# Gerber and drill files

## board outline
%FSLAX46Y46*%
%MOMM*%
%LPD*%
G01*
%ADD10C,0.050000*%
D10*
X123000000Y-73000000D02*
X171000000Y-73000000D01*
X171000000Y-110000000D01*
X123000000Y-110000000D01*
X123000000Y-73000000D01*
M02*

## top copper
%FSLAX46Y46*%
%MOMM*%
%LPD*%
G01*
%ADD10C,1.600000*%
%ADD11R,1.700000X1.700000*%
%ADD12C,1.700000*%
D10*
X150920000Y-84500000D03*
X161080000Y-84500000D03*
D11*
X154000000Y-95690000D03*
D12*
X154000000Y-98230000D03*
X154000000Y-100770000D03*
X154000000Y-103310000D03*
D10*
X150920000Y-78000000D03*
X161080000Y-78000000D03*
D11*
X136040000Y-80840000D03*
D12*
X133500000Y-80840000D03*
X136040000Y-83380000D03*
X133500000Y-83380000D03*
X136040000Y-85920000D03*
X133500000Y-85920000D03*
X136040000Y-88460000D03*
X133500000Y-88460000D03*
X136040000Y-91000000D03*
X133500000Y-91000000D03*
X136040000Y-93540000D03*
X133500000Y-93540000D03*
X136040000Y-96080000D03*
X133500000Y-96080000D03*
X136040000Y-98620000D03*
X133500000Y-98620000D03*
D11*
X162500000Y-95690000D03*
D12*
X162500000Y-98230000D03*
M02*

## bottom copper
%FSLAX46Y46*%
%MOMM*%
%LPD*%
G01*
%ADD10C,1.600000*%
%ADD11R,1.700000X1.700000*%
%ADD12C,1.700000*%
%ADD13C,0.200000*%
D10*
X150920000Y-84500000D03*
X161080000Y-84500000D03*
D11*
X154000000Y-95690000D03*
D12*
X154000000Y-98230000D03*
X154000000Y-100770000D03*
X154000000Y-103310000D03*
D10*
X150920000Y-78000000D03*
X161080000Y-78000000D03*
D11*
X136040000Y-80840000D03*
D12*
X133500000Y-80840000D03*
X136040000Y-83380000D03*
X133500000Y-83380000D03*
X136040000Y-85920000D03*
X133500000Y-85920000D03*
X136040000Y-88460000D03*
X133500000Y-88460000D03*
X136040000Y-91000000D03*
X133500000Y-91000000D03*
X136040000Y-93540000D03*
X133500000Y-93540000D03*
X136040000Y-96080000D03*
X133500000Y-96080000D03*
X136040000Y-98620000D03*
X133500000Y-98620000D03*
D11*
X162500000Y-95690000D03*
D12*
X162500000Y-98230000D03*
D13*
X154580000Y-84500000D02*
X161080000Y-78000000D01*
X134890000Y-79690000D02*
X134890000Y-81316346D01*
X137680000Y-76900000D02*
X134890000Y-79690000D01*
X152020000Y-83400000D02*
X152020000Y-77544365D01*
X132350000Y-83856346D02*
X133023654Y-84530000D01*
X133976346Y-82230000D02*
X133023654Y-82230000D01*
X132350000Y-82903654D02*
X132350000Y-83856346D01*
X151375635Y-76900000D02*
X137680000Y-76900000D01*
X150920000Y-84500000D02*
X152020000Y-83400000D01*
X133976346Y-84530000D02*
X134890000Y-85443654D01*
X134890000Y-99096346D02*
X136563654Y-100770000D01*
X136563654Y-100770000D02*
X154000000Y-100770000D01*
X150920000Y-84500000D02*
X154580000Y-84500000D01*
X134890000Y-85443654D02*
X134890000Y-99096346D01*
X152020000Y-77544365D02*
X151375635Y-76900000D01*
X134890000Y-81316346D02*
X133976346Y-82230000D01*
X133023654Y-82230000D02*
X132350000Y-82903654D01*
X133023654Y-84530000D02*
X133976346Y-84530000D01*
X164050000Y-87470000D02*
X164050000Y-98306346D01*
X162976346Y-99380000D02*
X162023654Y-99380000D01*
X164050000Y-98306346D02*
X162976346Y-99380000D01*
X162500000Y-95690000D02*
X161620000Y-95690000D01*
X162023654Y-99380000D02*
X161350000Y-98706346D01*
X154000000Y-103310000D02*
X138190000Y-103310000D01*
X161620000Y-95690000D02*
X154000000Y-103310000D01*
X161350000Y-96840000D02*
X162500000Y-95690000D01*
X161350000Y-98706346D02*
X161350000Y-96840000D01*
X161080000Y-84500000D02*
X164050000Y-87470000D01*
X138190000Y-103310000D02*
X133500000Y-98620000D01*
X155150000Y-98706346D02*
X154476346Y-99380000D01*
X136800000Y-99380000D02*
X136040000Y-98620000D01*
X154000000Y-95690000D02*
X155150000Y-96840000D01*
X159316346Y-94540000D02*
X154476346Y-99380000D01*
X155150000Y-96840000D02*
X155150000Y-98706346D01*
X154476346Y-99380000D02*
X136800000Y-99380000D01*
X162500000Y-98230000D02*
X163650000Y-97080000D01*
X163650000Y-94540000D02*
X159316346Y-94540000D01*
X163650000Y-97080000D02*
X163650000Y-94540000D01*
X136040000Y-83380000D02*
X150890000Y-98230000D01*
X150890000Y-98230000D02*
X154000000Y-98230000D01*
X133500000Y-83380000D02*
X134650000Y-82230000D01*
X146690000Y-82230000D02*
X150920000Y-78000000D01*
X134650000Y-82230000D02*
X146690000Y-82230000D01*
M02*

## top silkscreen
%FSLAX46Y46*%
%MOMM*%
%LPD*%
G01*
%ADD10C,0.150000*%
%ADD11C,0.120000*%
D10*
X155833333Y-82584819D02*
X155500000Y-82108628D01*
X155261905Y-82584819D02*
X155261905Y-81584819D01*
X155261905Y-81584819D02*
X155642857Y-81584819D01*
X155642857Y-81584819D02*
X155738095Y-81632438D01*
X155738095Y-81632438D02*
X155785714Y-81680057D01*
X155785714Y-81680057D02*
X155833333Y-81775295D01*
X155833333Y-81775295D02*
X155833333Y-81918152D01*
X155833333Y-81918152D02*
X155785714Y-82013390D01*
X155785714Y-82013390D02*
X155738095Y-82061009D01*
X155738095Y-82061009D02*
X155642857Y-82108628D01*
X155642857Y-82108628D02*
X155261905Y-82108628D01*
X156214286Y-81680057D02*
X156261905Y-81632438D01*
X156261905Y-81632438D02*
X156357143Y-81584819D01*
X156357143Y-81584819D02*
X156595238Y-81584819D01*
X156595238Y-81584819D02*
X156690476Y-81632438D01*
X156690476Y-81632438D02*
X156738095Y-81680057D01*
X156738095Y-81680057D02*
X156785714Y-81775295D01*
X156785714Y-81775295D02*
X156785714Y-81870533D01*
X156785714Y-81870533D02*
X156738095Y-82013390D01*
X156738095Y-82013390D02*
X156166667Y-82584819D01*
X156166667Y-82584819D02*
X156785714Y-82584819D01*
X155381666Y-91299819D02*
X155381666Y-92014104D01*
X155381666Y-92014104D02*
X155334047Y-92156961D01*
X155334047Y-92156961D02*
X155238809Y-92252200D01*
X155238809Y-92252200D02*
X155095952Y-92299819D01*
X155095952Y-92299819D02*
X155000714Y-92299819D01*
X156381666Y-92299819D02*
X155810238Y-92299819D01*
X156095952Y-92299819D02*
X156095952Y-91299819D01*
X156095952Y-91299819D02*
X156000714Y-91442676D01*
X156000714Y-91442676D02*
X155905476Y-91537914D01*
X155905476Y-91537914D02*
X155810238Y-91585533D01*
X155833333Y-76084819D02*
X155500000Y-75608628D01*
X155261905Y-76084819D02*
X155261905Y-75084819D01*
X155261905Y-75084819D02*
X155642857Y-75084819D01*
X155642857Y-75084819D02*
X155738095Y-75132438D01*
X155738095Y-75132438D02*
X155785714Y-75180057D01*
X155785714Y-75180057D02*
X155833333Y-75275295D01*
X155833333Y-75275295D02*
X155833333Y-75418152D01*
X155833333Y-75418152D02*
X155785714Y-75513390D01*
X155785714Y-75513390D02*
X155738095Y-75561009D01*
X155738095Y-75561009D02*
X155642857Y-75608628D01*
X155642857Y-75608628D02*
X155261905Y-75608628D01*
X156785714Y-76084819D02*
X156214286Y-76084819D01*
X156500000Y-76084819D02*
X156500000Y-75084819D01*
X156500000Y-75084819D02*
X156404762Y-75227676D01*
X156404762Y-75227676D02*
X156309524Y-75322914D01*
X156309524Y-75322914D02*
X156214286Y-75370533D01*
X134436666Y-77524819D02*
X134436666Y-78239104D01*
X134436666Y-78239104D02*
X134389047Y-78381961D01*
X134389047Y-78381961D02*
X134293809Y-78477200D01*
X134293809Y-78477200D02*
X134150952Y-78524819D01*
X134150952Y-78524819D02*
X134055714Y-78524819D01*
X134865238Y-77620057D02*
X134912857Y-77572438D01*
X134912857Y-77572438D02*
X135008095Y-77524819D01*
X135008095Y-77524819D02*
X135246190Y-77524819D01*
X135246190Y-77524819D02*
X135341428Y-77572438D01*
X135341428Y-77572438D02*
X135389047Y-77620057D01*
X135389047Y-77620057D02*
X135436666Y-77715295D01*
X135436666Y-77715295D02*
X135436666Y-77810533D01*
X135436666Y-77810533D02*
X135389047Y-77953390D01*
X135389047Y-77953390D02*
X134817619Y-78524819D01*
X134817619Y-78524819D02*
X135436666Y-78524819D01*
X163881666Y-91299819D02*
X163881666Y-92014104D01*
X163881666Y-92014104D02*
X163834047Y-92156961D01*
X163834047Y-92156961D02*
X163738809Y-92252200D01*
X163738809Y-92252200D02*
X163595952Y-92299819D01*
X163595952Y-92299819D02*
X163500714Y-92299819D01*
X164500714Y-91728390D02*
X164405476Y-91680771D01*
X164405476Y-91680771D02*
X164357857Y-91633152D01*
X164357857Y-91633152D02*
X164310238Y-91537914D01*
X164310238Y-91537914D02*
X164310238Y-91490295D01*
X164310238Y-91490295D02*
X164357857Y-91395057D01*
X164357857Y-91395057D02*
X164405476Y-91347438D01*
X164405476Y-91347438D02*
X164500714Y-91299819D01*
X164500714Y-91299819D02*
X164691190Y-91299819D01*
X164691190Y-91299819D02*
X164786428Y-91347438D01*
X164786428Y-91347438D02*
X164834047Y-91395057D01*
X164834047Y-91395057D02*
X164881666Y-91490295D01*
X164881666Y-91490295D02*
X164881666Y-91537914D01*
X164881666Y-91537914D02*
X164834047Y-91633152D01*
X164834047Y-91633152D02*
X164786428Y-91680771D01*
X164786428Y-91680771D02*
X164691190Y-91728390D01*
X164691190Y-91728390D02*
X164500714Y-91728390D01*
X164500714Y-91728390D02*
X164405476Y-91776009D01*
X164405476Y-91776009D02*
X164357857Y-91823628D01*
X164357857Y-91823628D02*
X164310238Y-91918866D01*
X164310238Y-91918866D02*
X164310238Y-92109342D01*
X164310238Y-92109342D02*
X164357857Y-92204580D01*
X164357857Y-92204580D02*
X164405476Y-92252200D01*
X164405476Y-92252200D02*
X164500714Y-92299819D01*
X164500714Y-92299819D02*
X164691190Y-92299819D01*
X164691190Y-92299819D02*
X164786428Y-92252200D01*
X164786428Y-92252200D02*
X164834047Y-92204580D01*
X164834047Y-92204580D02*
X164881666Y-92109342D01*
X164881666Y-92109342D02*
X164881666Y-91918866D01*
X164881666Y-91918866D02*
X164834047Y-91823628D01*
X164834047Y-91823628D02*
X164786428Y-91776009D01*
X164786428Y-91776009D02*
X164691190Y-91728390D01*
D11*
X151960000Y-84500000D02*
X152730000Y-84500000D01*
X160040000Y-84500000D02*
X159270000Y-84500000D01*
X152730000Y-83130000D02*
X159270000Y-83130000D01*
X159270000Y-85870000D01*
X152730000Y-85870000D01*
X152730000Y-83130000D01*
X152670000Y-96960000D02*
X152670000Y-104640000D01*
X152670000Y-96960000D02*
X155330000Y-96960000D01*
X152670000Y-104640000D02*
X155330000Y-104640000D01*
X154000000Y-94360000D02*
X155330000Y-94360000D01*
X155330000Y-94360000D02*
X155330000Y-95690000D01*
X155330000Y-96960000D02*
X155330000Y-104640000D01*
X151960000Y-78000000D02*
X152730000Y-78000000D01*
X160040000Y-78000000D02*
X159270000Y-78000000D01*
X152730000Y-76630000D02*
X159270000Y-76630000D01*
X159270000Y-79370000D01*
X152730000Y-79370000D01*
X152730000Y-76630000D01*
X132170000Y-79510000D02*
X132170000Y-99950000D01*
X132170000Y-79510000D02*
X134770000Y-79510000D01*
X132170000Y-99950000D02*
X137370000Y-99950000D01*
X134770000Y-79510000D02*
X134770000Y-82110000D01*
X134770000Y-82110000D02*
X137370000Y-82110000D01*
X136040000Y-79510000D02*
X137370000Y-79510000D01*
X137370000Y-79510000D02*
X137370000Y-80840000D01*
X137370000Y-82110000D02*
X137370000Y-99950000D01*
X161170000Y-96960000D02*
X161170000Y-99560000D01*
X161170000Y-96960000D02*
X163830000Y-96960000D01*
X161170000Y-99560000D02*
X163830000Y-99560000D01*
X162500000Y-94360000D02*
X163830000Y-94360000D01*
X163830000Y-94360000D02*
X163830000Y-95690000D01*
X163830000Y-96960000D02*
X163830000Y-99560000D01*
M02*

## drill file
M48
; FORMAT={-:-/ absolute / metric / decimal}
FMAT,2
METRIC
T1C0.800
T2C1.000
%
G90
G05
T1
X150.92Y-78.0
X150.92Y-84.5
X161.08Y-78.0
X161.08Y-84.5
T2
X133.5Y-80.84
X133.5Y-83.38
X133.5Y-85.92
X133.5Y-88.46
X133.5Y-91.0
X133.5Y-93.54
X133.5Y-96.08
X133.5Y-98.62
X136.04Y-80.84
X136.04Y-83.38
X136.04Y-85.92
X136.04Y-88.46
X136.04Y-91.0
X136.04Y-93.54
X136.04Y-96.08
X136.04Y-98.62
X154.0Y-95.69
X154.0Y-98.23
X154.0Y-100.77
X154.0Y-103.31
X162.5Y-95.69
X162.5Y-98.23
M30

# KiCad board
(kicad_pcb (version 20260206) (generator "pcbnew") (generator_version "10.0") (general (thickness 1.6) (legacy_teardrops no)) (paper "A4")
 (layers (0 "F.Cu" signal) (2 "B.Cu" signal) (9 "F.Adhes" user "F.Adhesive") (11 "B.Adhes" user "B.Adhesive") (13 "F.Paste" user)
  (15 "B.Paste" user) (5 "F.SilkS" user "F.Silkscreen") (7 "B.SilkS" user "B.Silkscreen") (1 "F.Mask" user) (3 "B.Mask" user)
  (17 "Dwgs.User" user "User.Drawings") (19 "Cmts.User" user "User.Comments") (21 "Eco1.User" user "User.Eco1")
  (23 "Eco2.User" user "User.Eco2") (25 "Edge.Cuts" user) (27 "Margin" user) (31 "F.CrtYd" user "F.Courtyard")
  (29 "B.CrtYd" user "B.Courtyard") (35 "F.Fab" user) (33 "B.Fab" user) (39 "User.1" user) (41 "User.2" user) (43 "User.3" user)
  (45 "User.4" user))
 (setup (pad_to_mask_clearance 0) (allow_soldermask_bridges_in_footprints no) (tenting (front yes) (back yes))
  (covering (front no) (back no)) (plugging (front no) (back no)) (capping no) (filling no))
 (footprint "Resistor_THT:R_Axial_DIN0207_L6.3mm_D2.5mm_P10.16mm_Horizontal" (layer "F.Cu") (at 150.92 84.5)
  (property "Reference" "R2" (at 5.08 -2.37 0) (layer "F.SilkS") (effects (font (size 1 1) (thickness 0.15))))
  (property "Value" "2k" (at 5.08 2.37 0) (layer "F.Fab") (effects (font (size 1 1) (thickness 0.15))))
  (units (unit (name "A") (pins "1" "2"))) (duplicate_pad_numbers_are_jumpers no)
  (fp_line (start 1.04 0) (end 1.81 0) (stroke (width 0.12) (type solid)) (layer "F.SilkS"))
  (fp_line (start 9.12 0) (end 8.35 0) (stroke (width 0.12) (type solid)) (layer "F.SilkS"))
  (fp_rect (start 1.81 -1.37) (end 8.35 1.37) (stroke (width 0.12) (type solid)) (fill no) (layer "F.SilkS"))
  (pad "1" thru_hole circle (at 0 0) (size 1.6 1.6) (drill 0.8) (layers "*.Cu" "*.Mask") (remove_unused_layers no) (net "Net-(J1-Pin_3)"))
  (pad "2" thru_hole circle (at 10.16 0) (size 1.6 1.6) (drill 0.8) (layers "*.Cu" "*.Mask") (remove_unused_layers no) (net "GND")))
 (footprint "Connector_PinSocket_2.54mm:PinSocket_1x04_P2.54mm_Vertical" (layer "F.Cu") (at 154 95.69)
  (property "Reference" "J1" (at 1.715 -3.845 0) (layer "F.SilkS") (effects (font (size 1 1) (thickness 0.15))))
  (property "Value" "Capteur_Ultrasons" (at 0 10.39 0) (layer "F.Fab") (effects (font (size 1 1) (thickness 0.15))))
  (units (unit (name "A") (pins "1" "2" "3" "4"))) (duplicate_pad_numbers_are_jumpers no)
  (fp_line (start -1.33 1.27) (end -1.33 8.95) (stroke (width 0.12) (type solid)) (layer "F.SilkS"))
  (fp_line (start -1.33 1.27) (end 1.33 1.27) (stroke (width 0.12) (type solid)) (layer "F.SilkS"))
  (fp_line (start -1.33 8.95) (end 1.33 8.95) (stroke (width 0.12) (type solid)) (layer "F.SilkS"))
  (fp_line (start 0 -1.33) (end 1.33 -1.33) (stroke (width 0.12) (type solid)) (layer "F.SilkS"))
  (fp_line (start 1.33 -1.33) (end 1.33 0) (stroke (width 0.12) (type solid)) (layer "F.SilkS"))
  (fp_line (start 1.33 1.27) (end 1.33 8.95) (stroke (width 0.12) (type solid)) (layer "F.SilkS"))
  (pad "1" thru_hole rect (at 0 0) (size 1.7 1.7) (drill 1) (layers "*.Cu" "*.Mask") (remove_unused_layers no) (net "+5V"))
  (pad "2" thru_hole circle (at 0 2.54) (size 1.7 1.7) (drill 1) (layers "*.Cu" "*.Mask") (remove_unused_layers no) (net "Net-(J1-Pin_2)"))
  (pad "3" thru_hole circle (at 0 5.08) (size 1.7 1.7) (drill 1) (layers "*.Cu" "*.Mask") (remove_unused_layers no) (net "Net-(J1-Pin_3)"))
  (pad "4" thru_hole circle (at 0 7.62) (size 1.7 1.7) (drill 1) (layers "*.Cu" "*.Mask") (remove_unused_layers no) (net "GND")))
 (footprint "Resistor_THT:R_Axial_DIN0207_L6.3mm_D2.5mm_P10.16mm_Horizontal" (layer "F.Cu") (at 150.92 78)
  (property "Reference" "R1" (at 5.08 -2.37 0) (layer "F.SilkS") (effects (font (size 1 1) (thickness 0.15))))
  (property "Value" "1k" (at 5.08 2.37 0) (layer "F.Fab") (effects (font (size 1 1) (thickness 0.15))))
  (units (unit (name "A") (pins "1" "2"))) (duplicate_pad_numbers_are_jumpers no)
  (fp_line (start 1.04 0) (end 1.81 0) (stroke (width 0.12) (type solid)) (layer "F.SilkS"))
  (fp_line (start 9.12 0) (end 8.35 0) (stroke (width 0.12) (type solid)) (layer "F.SilkS"))
  (fp_rect (start 1.81 -1.37) (end 8.35 1.37) (stroke (width 0.12) (type solid)) (fill no) (layer "F.SilkS"))
  (pad "1" thru_hole circle (at 0 0) (size 1.6 1.6) (drill 0.8) (layers "*.Cu" "*.Mask") (remove_unused_layers no) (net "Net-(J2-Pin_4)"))
  (pad "2" thru_hole circle (at 10.16 0) (size 1.6 1.6) (drill 0.8) (layers "*.Cu" "*.Mask") (remove_unused_layers no)
   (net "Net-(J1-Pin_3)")))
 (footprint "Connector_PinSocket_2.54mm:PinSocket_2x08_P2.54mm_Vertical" (layer "F.Cu") (at 136.04 80.84)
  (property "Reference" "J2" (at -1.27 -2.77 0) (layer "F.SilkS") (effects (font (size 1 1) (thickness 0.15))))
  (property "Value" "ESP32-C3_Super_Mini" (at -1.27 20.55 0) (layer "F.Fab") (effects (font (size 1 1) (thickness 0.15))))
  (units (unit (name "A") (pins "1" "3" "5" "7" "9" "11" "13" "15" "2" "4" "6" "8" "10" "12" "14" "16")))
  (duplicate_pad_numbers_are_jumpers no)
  (fp_line (start -3.87 -1.33) (end -3.87 19.11) (stroke (width 0.12) (type solid)) (layer "F.SilkS"))
  (fp_line (start -3.87 -1.33) (end -1.27 -1.33) (stroke (width 0.12) (type solid)) (layer "F.SilkS"))
  (fp_line (start -3.87 19.11) (end 1.33 19.11) (stroke (width 0.12) (type solid)) (layer "F.SilkS"))
  (fp_line (start -1.27 -1.33) (end -1.27 1.27) (stroke (width 0.12) (type solid)) (layer "F.SilkS"))
  (fp_line (start -1.27 1.27) (end 1.33 1.27) (stroke (width 0.12) (type solid)) (layer "F.SilkS"))
  (fp_line (start 0 -1.33) (end 1.33 -1.33) (stroke (width 0.12) (type solid)) (layer "F.SilkS"))
  (fp_line (start 1.33 -1.33) (end 1.33 0) (stroke (width 0.12) (type solid)) (layer "F.SilkS"))
  (fp_line (start 1.33 1.27) (end 1.33 19.11) (stroke (width 0.12) (type solid)) (layer "F.SilkS"))
  (pad "1" thru_hole rect (at 0 0) (size 1.7 1.7) (drill 1) (layers "*.Cu" "*.Mask") (remove_unused_layers no)
   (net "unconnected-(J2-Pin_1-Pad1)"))
  (pad "2" thru_hole circle (at -2.54 0) (size 1.7 1.7) (drill 1) (layers "*.Cu" "*.Mask") (remove_unused_layers no)
   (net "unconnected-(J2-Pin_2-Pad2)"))
  (pad "3" thru_hole circle (at 0 2.54) (size 1.7 1.7) (drill 1) (layers "*.Cu" "*.Mask") (remove_unused_layers no) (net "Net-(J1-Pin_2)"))
  (pad "4" thru_hole circle (at -2.54 2.54) (size 1.7 1.7) (drill 1) (layers "*.Cu" "*.Mask") (remove_unused_layers no)
   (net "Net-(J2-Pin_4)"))
  (pad "5" thru_hole circle (at 0 5.08) (size 1.7 1.7) (drill 1) (layers "*.Cu" "*.Mask") (remove_unused_layers no)
   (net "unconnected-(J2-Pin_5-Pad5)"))
  (pad "6" thru_hole circle (at -2.54 5.08) (size 1.7 1.7) (drill 1) (layers "*.Cu" "*.Mask") (remove_unused_layers no)
   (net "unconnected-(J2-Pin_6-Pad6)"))
  (pad "7" thru_hole circle (at 0 7.62) (size 1.7 1.7) (drill 1) (layers "*.Cu" "*.Mask") (remove_unused_layers no)
   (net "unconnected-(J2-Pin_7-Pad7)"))
  (pad "8" thru_hole circle (at -2.54 7.62) (size 1.7 1.7) (drill 1) (layers "*.Cu" "*.Mask") (remove_unused_layers no)
   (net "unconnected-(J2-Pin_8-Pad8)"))
  (pad "9" thru_hole circle (at 0 10.16) (size 1.7 1.7) (drill 1) (layers "*.Cu" "*.Mask") (remove_unused_layers no)
   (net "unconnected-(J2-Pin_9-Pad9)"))
  (pad "10" thru_hole circle (at -2.54 10.16) (size 1.7 1.7) (drill 1) (layers "*.Cu" "*.Mask") (remove_unused_layers no)
   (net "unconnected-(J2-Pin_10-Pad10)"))
  (pad "11" thru_hole circle (at 0 12.7) (size 1.7 1.7) (drill 1) (layers "*.Cu" "*.Mask") (remove_unused_layers no)
   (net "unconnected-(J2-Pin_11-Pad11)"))
  (pad "12" thru_hole circle (at -2.54 12.7) (size 1.7 1.7) (drill 1) (layers "*.Cu" "*.Mask") (remove_unused_layers no)
   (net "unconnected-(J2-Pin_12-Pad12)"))
  (pad "13" thru_hole circle (at 0 15.24) (size 1.7 1.7) (drill 1) (layers "*.Cu" "*.Mask") (remove_unused_layers no)
   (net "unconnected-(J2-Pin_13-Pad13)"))
  (pad "14" thru_hole circle (at -2.54 15.24) (size 1.7 1.7) (drill 1) (layers "*.Cu" "*.Mask") (remove_unused_layers no)
   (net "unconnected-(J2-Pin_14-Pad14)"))
  (pad "15" thru_hole circle (at 0 17.78) (size 1.7 1.7) (drill 1) (layers "*.Cu" "*.Mask") (remove_unused_layers no) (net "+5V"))
  (pad "16" thru_hole circle (at -2.54 17.78) (size 1.7 1.7) (drill 1) (layers "*.Cu" "*.Mask") (remove_unused_layers no) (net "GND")))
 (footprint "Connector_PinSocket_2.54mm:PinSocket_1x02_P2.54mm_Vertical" (layer "F.Cu") (at 162.5 95.69)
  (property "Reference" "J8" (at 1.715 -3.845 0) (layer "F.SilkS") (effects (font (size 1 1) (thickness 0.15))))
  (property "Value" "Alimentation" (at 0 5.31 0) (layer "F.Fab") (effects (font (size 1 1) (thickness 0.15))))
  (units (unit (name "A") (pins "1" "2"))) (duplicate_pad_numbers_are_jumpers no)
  (fp_line (start -1.33 1.27) (end -1.33 3.87) (stroke (width 0.12) (type solid)) (layer "F.SilkS"))
  (fp_line (start -1.33 1.27) (end 1.33 1.27) (stroke (width 0.12) (type solid)) (layer "F.SilkS"))
  (fp_line (start -1.33 3.87) (end 1.33 3.87) (stroke (width 0.12) (type solid)) (layer "F.SilkS"))
  (fp_line (start 0 -1.33) (end 1.33 -1.33) (stroke (width 0.12) (type solid)) (layer "F.SilkS"))
  (fp_line (start 1.33 -1.33) (end 1.33 0) (stroke (width 0.12) (type solid)) (layer "F.SilkS"))
  (fp_line (start 1.33 1.27) (end 1.33 3.87) (stroke (width 0.12) (type solid)) (layer "F.SilkS"))
  (pad "1" thru_hole rect (at 0 0) (size 1.7 1.7) (drill 1) (layers "*.Cu" "*.Mask") (remove_unused_layers no) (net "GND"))
  (pad "2" thru_hole circle (at 0 2.54) (size 1.7 1.7) (drill 1) (layers "*.Cu" "*.Mask") (remove_unused_layers no) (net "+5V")))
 (gr_rect (start 123 73) (end 171 110) (stroke (width 0.05) (type default)) (fill no) (layer "Edge.Cuts"))
 (segment (start 154.58 84.5) (end 161.08 78) (width 0.2) (layer "B.Cu") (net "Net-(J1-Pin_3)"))
 (segment (start 134.89 79.69) (end 134.89 81.316346) (width 0.2) (layer "B.Cu") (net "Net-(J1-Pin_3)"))
 (segment (start 137.68 76.9) (end 134.89 79.69) (width 0.2) (layer "B.Cu") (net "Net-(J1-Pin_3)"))
 (segment (start 152.02 83.4) (end 152.02 77.544365) (width 0.2) (layer "B.Cu") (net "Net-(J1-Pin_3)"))
 (segment (start 132.35 83.856346) (end 133.023654 84.53) (width 0.2) (layer "B.Cu") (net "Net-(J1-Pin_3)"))
 (segment (start 133.976346 82.23) (end 133.023654 82.23) (width 0.2) (layer "B.Cu") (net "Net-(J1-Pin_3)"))
 (segment (start 132.35 82.903654) (end 132.35 83.856346) (width 0.2) (layer "B.Cu") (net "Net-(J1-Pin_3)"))
 (segment (start 151.375635 76.9) (end 137.68 76.9) (width 0.2) (layer "B.Cu") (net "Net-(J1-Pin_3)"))
 (segment (start 150.92 84.5) (end 152.02 83.4) (width 0.2) (layer "B.Cu") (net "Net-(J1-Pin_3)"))
 (segment (start 133.976346 84.53) (end 134.89 85.443654) (width 0.2) (layer "B.Cu") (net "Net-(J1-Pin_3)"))
 (segment (start 134.89 99.096346) (end 136.563654 100.77) (width 0.2) (layer "B.Cu") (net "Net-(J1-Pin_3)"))
 (segment (start 136.563654 100.77) (end 154 100.77) (width 0.2) (layer "B.Cu") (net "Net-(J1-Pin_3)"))
 (segment (start 150.92 84.5) (end 154.58 84.5) (width 0.2) (layer "B.Cu") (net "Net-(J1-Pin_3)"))
 (segment (start 134.89 85.443654) (end 134.89 99.096346) (width 0.2) (layer "B.Cu") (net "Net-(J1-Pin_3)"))
 (segment (start 152.02 77.544365) (end 151.375635 76.9) (width 0.2) (layer "B.Cu") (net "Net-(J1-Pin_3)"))
 (segment (start 134.89 81.316346) (end 133.976346 82.23) (width 0.2) (layer "B.Cu") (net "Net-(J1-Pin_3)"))
 (segment (start 133.023654 82.23) (end 132.35 82.903654) (width 0.2) (layer "B.Cu") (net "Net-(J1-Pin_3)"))
 (segment (start 133.023654 84.53) (end 133.976346 84.53) (width 0.2) (layer "B.Cu") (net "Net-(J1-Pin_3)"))
 (segment (start 164.05 87.47) (end 164.05 98.306346) (width 0.2) (layer "B.Cu") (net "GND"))
 (segment (start 162.976346 99.38) (end 162.023654 99.38) (width 0.2) (layer "B.Cu") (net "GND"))
 (segment (start 164.05 98.306346) (end 162.976346 99.38) (width 0.2) (layer "B.Cu") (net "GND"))
 (segment (start 162.5 95.69) (end 161.62 95.69) (width 0.2) (layer "B.Cu") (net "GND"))
 (segment (start 162.023654 99.38) (end 161.35 98.706346) (width 0.2) (layer "B.Cu") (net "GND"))
 (segment (start 154 103.31) (end 138.19 103.31) (width 0.2) (layer "B.Cu") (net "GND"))
 (segment (start 161.62 95.69) (end 154 103.31) (width 0.2) (layer "B.Cu") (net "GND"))
 (segment (start 161.35 96.84) (end 162.5 95.69) (width 0.2) (layer "B.Cu") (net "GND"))
 (segment (start 161.35 98.706346) (end 161.35 96.84) (width 0.2) (layer "B.Cu") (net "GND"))
 (segment (start 161.08 84.5) (end 164.05 87.47) (width 0.2) (layer "B.Cu") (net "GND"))
 (segment (start 138.19 103.31) (end 133.5 98.62) (width 0.2) (layer "B.Cu") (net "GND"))
 (segment (start 155.15 98.706346) (end 154.476346 99.38) (width 0.2) (layer "B.Cu") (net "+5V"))
 (segment (start 136.8 99.38) (end 136.04 98.62) (width 0.2) (layer "B.Cu") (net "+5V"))
 (segment (start 154 95.69) (end 155.15 96.84) (width 0.2) (layer "B.Cu") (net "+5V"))
 (segment (start 159.316346 94.54) (end 154.476346 99.38) (width 0.2) (layer "B.Cu") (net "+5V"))
 (segment (start 155.15 96.84) (end 155.15 98.706346) (width 0.2) (layer "B.Cu") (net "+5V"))
 (segment (start 154.476346 99.38) (end 136.8 99.38) (width 0.2) (layer "B.Cu") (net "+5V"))
 (segment (start 162.5 98.23) (end 163.65 97.08) (width 0.2) (layer "B.Cu") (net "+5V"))
 (segment (start 163.65 94.54) (end 159.316346 94.54) (width 0.2) (layer "B.Cu") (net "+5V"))
 (segment (start 163.65 97.08) (end 163.65 94.54) (width 0.2) (layer "B.Cu") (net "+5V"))
 (segment (start 136.04 83.38) (end 150.89 98.23) (width 0.2) (layer "B.Cu") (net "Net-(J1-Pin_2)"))
 (segment (start 150.89 98.23) (end 154 98.23) (width 0.2) (layer "B.Cu") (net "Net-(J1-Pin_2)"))
 (segment (start 133.5 83.38) (end 134.65 82.23) (width 0.2) (layer "B.Cu") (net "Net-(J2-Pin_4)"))
 (segment (start 146.69 82.23) (end 150.92 78) (width 0.2) (layer "B.Cu") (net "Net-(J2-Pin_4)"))
 (segment (start 134.65 82.23) (end 146.69 82.23) (width 0.2) (layer "B.Cu") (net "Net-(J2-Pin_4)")))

